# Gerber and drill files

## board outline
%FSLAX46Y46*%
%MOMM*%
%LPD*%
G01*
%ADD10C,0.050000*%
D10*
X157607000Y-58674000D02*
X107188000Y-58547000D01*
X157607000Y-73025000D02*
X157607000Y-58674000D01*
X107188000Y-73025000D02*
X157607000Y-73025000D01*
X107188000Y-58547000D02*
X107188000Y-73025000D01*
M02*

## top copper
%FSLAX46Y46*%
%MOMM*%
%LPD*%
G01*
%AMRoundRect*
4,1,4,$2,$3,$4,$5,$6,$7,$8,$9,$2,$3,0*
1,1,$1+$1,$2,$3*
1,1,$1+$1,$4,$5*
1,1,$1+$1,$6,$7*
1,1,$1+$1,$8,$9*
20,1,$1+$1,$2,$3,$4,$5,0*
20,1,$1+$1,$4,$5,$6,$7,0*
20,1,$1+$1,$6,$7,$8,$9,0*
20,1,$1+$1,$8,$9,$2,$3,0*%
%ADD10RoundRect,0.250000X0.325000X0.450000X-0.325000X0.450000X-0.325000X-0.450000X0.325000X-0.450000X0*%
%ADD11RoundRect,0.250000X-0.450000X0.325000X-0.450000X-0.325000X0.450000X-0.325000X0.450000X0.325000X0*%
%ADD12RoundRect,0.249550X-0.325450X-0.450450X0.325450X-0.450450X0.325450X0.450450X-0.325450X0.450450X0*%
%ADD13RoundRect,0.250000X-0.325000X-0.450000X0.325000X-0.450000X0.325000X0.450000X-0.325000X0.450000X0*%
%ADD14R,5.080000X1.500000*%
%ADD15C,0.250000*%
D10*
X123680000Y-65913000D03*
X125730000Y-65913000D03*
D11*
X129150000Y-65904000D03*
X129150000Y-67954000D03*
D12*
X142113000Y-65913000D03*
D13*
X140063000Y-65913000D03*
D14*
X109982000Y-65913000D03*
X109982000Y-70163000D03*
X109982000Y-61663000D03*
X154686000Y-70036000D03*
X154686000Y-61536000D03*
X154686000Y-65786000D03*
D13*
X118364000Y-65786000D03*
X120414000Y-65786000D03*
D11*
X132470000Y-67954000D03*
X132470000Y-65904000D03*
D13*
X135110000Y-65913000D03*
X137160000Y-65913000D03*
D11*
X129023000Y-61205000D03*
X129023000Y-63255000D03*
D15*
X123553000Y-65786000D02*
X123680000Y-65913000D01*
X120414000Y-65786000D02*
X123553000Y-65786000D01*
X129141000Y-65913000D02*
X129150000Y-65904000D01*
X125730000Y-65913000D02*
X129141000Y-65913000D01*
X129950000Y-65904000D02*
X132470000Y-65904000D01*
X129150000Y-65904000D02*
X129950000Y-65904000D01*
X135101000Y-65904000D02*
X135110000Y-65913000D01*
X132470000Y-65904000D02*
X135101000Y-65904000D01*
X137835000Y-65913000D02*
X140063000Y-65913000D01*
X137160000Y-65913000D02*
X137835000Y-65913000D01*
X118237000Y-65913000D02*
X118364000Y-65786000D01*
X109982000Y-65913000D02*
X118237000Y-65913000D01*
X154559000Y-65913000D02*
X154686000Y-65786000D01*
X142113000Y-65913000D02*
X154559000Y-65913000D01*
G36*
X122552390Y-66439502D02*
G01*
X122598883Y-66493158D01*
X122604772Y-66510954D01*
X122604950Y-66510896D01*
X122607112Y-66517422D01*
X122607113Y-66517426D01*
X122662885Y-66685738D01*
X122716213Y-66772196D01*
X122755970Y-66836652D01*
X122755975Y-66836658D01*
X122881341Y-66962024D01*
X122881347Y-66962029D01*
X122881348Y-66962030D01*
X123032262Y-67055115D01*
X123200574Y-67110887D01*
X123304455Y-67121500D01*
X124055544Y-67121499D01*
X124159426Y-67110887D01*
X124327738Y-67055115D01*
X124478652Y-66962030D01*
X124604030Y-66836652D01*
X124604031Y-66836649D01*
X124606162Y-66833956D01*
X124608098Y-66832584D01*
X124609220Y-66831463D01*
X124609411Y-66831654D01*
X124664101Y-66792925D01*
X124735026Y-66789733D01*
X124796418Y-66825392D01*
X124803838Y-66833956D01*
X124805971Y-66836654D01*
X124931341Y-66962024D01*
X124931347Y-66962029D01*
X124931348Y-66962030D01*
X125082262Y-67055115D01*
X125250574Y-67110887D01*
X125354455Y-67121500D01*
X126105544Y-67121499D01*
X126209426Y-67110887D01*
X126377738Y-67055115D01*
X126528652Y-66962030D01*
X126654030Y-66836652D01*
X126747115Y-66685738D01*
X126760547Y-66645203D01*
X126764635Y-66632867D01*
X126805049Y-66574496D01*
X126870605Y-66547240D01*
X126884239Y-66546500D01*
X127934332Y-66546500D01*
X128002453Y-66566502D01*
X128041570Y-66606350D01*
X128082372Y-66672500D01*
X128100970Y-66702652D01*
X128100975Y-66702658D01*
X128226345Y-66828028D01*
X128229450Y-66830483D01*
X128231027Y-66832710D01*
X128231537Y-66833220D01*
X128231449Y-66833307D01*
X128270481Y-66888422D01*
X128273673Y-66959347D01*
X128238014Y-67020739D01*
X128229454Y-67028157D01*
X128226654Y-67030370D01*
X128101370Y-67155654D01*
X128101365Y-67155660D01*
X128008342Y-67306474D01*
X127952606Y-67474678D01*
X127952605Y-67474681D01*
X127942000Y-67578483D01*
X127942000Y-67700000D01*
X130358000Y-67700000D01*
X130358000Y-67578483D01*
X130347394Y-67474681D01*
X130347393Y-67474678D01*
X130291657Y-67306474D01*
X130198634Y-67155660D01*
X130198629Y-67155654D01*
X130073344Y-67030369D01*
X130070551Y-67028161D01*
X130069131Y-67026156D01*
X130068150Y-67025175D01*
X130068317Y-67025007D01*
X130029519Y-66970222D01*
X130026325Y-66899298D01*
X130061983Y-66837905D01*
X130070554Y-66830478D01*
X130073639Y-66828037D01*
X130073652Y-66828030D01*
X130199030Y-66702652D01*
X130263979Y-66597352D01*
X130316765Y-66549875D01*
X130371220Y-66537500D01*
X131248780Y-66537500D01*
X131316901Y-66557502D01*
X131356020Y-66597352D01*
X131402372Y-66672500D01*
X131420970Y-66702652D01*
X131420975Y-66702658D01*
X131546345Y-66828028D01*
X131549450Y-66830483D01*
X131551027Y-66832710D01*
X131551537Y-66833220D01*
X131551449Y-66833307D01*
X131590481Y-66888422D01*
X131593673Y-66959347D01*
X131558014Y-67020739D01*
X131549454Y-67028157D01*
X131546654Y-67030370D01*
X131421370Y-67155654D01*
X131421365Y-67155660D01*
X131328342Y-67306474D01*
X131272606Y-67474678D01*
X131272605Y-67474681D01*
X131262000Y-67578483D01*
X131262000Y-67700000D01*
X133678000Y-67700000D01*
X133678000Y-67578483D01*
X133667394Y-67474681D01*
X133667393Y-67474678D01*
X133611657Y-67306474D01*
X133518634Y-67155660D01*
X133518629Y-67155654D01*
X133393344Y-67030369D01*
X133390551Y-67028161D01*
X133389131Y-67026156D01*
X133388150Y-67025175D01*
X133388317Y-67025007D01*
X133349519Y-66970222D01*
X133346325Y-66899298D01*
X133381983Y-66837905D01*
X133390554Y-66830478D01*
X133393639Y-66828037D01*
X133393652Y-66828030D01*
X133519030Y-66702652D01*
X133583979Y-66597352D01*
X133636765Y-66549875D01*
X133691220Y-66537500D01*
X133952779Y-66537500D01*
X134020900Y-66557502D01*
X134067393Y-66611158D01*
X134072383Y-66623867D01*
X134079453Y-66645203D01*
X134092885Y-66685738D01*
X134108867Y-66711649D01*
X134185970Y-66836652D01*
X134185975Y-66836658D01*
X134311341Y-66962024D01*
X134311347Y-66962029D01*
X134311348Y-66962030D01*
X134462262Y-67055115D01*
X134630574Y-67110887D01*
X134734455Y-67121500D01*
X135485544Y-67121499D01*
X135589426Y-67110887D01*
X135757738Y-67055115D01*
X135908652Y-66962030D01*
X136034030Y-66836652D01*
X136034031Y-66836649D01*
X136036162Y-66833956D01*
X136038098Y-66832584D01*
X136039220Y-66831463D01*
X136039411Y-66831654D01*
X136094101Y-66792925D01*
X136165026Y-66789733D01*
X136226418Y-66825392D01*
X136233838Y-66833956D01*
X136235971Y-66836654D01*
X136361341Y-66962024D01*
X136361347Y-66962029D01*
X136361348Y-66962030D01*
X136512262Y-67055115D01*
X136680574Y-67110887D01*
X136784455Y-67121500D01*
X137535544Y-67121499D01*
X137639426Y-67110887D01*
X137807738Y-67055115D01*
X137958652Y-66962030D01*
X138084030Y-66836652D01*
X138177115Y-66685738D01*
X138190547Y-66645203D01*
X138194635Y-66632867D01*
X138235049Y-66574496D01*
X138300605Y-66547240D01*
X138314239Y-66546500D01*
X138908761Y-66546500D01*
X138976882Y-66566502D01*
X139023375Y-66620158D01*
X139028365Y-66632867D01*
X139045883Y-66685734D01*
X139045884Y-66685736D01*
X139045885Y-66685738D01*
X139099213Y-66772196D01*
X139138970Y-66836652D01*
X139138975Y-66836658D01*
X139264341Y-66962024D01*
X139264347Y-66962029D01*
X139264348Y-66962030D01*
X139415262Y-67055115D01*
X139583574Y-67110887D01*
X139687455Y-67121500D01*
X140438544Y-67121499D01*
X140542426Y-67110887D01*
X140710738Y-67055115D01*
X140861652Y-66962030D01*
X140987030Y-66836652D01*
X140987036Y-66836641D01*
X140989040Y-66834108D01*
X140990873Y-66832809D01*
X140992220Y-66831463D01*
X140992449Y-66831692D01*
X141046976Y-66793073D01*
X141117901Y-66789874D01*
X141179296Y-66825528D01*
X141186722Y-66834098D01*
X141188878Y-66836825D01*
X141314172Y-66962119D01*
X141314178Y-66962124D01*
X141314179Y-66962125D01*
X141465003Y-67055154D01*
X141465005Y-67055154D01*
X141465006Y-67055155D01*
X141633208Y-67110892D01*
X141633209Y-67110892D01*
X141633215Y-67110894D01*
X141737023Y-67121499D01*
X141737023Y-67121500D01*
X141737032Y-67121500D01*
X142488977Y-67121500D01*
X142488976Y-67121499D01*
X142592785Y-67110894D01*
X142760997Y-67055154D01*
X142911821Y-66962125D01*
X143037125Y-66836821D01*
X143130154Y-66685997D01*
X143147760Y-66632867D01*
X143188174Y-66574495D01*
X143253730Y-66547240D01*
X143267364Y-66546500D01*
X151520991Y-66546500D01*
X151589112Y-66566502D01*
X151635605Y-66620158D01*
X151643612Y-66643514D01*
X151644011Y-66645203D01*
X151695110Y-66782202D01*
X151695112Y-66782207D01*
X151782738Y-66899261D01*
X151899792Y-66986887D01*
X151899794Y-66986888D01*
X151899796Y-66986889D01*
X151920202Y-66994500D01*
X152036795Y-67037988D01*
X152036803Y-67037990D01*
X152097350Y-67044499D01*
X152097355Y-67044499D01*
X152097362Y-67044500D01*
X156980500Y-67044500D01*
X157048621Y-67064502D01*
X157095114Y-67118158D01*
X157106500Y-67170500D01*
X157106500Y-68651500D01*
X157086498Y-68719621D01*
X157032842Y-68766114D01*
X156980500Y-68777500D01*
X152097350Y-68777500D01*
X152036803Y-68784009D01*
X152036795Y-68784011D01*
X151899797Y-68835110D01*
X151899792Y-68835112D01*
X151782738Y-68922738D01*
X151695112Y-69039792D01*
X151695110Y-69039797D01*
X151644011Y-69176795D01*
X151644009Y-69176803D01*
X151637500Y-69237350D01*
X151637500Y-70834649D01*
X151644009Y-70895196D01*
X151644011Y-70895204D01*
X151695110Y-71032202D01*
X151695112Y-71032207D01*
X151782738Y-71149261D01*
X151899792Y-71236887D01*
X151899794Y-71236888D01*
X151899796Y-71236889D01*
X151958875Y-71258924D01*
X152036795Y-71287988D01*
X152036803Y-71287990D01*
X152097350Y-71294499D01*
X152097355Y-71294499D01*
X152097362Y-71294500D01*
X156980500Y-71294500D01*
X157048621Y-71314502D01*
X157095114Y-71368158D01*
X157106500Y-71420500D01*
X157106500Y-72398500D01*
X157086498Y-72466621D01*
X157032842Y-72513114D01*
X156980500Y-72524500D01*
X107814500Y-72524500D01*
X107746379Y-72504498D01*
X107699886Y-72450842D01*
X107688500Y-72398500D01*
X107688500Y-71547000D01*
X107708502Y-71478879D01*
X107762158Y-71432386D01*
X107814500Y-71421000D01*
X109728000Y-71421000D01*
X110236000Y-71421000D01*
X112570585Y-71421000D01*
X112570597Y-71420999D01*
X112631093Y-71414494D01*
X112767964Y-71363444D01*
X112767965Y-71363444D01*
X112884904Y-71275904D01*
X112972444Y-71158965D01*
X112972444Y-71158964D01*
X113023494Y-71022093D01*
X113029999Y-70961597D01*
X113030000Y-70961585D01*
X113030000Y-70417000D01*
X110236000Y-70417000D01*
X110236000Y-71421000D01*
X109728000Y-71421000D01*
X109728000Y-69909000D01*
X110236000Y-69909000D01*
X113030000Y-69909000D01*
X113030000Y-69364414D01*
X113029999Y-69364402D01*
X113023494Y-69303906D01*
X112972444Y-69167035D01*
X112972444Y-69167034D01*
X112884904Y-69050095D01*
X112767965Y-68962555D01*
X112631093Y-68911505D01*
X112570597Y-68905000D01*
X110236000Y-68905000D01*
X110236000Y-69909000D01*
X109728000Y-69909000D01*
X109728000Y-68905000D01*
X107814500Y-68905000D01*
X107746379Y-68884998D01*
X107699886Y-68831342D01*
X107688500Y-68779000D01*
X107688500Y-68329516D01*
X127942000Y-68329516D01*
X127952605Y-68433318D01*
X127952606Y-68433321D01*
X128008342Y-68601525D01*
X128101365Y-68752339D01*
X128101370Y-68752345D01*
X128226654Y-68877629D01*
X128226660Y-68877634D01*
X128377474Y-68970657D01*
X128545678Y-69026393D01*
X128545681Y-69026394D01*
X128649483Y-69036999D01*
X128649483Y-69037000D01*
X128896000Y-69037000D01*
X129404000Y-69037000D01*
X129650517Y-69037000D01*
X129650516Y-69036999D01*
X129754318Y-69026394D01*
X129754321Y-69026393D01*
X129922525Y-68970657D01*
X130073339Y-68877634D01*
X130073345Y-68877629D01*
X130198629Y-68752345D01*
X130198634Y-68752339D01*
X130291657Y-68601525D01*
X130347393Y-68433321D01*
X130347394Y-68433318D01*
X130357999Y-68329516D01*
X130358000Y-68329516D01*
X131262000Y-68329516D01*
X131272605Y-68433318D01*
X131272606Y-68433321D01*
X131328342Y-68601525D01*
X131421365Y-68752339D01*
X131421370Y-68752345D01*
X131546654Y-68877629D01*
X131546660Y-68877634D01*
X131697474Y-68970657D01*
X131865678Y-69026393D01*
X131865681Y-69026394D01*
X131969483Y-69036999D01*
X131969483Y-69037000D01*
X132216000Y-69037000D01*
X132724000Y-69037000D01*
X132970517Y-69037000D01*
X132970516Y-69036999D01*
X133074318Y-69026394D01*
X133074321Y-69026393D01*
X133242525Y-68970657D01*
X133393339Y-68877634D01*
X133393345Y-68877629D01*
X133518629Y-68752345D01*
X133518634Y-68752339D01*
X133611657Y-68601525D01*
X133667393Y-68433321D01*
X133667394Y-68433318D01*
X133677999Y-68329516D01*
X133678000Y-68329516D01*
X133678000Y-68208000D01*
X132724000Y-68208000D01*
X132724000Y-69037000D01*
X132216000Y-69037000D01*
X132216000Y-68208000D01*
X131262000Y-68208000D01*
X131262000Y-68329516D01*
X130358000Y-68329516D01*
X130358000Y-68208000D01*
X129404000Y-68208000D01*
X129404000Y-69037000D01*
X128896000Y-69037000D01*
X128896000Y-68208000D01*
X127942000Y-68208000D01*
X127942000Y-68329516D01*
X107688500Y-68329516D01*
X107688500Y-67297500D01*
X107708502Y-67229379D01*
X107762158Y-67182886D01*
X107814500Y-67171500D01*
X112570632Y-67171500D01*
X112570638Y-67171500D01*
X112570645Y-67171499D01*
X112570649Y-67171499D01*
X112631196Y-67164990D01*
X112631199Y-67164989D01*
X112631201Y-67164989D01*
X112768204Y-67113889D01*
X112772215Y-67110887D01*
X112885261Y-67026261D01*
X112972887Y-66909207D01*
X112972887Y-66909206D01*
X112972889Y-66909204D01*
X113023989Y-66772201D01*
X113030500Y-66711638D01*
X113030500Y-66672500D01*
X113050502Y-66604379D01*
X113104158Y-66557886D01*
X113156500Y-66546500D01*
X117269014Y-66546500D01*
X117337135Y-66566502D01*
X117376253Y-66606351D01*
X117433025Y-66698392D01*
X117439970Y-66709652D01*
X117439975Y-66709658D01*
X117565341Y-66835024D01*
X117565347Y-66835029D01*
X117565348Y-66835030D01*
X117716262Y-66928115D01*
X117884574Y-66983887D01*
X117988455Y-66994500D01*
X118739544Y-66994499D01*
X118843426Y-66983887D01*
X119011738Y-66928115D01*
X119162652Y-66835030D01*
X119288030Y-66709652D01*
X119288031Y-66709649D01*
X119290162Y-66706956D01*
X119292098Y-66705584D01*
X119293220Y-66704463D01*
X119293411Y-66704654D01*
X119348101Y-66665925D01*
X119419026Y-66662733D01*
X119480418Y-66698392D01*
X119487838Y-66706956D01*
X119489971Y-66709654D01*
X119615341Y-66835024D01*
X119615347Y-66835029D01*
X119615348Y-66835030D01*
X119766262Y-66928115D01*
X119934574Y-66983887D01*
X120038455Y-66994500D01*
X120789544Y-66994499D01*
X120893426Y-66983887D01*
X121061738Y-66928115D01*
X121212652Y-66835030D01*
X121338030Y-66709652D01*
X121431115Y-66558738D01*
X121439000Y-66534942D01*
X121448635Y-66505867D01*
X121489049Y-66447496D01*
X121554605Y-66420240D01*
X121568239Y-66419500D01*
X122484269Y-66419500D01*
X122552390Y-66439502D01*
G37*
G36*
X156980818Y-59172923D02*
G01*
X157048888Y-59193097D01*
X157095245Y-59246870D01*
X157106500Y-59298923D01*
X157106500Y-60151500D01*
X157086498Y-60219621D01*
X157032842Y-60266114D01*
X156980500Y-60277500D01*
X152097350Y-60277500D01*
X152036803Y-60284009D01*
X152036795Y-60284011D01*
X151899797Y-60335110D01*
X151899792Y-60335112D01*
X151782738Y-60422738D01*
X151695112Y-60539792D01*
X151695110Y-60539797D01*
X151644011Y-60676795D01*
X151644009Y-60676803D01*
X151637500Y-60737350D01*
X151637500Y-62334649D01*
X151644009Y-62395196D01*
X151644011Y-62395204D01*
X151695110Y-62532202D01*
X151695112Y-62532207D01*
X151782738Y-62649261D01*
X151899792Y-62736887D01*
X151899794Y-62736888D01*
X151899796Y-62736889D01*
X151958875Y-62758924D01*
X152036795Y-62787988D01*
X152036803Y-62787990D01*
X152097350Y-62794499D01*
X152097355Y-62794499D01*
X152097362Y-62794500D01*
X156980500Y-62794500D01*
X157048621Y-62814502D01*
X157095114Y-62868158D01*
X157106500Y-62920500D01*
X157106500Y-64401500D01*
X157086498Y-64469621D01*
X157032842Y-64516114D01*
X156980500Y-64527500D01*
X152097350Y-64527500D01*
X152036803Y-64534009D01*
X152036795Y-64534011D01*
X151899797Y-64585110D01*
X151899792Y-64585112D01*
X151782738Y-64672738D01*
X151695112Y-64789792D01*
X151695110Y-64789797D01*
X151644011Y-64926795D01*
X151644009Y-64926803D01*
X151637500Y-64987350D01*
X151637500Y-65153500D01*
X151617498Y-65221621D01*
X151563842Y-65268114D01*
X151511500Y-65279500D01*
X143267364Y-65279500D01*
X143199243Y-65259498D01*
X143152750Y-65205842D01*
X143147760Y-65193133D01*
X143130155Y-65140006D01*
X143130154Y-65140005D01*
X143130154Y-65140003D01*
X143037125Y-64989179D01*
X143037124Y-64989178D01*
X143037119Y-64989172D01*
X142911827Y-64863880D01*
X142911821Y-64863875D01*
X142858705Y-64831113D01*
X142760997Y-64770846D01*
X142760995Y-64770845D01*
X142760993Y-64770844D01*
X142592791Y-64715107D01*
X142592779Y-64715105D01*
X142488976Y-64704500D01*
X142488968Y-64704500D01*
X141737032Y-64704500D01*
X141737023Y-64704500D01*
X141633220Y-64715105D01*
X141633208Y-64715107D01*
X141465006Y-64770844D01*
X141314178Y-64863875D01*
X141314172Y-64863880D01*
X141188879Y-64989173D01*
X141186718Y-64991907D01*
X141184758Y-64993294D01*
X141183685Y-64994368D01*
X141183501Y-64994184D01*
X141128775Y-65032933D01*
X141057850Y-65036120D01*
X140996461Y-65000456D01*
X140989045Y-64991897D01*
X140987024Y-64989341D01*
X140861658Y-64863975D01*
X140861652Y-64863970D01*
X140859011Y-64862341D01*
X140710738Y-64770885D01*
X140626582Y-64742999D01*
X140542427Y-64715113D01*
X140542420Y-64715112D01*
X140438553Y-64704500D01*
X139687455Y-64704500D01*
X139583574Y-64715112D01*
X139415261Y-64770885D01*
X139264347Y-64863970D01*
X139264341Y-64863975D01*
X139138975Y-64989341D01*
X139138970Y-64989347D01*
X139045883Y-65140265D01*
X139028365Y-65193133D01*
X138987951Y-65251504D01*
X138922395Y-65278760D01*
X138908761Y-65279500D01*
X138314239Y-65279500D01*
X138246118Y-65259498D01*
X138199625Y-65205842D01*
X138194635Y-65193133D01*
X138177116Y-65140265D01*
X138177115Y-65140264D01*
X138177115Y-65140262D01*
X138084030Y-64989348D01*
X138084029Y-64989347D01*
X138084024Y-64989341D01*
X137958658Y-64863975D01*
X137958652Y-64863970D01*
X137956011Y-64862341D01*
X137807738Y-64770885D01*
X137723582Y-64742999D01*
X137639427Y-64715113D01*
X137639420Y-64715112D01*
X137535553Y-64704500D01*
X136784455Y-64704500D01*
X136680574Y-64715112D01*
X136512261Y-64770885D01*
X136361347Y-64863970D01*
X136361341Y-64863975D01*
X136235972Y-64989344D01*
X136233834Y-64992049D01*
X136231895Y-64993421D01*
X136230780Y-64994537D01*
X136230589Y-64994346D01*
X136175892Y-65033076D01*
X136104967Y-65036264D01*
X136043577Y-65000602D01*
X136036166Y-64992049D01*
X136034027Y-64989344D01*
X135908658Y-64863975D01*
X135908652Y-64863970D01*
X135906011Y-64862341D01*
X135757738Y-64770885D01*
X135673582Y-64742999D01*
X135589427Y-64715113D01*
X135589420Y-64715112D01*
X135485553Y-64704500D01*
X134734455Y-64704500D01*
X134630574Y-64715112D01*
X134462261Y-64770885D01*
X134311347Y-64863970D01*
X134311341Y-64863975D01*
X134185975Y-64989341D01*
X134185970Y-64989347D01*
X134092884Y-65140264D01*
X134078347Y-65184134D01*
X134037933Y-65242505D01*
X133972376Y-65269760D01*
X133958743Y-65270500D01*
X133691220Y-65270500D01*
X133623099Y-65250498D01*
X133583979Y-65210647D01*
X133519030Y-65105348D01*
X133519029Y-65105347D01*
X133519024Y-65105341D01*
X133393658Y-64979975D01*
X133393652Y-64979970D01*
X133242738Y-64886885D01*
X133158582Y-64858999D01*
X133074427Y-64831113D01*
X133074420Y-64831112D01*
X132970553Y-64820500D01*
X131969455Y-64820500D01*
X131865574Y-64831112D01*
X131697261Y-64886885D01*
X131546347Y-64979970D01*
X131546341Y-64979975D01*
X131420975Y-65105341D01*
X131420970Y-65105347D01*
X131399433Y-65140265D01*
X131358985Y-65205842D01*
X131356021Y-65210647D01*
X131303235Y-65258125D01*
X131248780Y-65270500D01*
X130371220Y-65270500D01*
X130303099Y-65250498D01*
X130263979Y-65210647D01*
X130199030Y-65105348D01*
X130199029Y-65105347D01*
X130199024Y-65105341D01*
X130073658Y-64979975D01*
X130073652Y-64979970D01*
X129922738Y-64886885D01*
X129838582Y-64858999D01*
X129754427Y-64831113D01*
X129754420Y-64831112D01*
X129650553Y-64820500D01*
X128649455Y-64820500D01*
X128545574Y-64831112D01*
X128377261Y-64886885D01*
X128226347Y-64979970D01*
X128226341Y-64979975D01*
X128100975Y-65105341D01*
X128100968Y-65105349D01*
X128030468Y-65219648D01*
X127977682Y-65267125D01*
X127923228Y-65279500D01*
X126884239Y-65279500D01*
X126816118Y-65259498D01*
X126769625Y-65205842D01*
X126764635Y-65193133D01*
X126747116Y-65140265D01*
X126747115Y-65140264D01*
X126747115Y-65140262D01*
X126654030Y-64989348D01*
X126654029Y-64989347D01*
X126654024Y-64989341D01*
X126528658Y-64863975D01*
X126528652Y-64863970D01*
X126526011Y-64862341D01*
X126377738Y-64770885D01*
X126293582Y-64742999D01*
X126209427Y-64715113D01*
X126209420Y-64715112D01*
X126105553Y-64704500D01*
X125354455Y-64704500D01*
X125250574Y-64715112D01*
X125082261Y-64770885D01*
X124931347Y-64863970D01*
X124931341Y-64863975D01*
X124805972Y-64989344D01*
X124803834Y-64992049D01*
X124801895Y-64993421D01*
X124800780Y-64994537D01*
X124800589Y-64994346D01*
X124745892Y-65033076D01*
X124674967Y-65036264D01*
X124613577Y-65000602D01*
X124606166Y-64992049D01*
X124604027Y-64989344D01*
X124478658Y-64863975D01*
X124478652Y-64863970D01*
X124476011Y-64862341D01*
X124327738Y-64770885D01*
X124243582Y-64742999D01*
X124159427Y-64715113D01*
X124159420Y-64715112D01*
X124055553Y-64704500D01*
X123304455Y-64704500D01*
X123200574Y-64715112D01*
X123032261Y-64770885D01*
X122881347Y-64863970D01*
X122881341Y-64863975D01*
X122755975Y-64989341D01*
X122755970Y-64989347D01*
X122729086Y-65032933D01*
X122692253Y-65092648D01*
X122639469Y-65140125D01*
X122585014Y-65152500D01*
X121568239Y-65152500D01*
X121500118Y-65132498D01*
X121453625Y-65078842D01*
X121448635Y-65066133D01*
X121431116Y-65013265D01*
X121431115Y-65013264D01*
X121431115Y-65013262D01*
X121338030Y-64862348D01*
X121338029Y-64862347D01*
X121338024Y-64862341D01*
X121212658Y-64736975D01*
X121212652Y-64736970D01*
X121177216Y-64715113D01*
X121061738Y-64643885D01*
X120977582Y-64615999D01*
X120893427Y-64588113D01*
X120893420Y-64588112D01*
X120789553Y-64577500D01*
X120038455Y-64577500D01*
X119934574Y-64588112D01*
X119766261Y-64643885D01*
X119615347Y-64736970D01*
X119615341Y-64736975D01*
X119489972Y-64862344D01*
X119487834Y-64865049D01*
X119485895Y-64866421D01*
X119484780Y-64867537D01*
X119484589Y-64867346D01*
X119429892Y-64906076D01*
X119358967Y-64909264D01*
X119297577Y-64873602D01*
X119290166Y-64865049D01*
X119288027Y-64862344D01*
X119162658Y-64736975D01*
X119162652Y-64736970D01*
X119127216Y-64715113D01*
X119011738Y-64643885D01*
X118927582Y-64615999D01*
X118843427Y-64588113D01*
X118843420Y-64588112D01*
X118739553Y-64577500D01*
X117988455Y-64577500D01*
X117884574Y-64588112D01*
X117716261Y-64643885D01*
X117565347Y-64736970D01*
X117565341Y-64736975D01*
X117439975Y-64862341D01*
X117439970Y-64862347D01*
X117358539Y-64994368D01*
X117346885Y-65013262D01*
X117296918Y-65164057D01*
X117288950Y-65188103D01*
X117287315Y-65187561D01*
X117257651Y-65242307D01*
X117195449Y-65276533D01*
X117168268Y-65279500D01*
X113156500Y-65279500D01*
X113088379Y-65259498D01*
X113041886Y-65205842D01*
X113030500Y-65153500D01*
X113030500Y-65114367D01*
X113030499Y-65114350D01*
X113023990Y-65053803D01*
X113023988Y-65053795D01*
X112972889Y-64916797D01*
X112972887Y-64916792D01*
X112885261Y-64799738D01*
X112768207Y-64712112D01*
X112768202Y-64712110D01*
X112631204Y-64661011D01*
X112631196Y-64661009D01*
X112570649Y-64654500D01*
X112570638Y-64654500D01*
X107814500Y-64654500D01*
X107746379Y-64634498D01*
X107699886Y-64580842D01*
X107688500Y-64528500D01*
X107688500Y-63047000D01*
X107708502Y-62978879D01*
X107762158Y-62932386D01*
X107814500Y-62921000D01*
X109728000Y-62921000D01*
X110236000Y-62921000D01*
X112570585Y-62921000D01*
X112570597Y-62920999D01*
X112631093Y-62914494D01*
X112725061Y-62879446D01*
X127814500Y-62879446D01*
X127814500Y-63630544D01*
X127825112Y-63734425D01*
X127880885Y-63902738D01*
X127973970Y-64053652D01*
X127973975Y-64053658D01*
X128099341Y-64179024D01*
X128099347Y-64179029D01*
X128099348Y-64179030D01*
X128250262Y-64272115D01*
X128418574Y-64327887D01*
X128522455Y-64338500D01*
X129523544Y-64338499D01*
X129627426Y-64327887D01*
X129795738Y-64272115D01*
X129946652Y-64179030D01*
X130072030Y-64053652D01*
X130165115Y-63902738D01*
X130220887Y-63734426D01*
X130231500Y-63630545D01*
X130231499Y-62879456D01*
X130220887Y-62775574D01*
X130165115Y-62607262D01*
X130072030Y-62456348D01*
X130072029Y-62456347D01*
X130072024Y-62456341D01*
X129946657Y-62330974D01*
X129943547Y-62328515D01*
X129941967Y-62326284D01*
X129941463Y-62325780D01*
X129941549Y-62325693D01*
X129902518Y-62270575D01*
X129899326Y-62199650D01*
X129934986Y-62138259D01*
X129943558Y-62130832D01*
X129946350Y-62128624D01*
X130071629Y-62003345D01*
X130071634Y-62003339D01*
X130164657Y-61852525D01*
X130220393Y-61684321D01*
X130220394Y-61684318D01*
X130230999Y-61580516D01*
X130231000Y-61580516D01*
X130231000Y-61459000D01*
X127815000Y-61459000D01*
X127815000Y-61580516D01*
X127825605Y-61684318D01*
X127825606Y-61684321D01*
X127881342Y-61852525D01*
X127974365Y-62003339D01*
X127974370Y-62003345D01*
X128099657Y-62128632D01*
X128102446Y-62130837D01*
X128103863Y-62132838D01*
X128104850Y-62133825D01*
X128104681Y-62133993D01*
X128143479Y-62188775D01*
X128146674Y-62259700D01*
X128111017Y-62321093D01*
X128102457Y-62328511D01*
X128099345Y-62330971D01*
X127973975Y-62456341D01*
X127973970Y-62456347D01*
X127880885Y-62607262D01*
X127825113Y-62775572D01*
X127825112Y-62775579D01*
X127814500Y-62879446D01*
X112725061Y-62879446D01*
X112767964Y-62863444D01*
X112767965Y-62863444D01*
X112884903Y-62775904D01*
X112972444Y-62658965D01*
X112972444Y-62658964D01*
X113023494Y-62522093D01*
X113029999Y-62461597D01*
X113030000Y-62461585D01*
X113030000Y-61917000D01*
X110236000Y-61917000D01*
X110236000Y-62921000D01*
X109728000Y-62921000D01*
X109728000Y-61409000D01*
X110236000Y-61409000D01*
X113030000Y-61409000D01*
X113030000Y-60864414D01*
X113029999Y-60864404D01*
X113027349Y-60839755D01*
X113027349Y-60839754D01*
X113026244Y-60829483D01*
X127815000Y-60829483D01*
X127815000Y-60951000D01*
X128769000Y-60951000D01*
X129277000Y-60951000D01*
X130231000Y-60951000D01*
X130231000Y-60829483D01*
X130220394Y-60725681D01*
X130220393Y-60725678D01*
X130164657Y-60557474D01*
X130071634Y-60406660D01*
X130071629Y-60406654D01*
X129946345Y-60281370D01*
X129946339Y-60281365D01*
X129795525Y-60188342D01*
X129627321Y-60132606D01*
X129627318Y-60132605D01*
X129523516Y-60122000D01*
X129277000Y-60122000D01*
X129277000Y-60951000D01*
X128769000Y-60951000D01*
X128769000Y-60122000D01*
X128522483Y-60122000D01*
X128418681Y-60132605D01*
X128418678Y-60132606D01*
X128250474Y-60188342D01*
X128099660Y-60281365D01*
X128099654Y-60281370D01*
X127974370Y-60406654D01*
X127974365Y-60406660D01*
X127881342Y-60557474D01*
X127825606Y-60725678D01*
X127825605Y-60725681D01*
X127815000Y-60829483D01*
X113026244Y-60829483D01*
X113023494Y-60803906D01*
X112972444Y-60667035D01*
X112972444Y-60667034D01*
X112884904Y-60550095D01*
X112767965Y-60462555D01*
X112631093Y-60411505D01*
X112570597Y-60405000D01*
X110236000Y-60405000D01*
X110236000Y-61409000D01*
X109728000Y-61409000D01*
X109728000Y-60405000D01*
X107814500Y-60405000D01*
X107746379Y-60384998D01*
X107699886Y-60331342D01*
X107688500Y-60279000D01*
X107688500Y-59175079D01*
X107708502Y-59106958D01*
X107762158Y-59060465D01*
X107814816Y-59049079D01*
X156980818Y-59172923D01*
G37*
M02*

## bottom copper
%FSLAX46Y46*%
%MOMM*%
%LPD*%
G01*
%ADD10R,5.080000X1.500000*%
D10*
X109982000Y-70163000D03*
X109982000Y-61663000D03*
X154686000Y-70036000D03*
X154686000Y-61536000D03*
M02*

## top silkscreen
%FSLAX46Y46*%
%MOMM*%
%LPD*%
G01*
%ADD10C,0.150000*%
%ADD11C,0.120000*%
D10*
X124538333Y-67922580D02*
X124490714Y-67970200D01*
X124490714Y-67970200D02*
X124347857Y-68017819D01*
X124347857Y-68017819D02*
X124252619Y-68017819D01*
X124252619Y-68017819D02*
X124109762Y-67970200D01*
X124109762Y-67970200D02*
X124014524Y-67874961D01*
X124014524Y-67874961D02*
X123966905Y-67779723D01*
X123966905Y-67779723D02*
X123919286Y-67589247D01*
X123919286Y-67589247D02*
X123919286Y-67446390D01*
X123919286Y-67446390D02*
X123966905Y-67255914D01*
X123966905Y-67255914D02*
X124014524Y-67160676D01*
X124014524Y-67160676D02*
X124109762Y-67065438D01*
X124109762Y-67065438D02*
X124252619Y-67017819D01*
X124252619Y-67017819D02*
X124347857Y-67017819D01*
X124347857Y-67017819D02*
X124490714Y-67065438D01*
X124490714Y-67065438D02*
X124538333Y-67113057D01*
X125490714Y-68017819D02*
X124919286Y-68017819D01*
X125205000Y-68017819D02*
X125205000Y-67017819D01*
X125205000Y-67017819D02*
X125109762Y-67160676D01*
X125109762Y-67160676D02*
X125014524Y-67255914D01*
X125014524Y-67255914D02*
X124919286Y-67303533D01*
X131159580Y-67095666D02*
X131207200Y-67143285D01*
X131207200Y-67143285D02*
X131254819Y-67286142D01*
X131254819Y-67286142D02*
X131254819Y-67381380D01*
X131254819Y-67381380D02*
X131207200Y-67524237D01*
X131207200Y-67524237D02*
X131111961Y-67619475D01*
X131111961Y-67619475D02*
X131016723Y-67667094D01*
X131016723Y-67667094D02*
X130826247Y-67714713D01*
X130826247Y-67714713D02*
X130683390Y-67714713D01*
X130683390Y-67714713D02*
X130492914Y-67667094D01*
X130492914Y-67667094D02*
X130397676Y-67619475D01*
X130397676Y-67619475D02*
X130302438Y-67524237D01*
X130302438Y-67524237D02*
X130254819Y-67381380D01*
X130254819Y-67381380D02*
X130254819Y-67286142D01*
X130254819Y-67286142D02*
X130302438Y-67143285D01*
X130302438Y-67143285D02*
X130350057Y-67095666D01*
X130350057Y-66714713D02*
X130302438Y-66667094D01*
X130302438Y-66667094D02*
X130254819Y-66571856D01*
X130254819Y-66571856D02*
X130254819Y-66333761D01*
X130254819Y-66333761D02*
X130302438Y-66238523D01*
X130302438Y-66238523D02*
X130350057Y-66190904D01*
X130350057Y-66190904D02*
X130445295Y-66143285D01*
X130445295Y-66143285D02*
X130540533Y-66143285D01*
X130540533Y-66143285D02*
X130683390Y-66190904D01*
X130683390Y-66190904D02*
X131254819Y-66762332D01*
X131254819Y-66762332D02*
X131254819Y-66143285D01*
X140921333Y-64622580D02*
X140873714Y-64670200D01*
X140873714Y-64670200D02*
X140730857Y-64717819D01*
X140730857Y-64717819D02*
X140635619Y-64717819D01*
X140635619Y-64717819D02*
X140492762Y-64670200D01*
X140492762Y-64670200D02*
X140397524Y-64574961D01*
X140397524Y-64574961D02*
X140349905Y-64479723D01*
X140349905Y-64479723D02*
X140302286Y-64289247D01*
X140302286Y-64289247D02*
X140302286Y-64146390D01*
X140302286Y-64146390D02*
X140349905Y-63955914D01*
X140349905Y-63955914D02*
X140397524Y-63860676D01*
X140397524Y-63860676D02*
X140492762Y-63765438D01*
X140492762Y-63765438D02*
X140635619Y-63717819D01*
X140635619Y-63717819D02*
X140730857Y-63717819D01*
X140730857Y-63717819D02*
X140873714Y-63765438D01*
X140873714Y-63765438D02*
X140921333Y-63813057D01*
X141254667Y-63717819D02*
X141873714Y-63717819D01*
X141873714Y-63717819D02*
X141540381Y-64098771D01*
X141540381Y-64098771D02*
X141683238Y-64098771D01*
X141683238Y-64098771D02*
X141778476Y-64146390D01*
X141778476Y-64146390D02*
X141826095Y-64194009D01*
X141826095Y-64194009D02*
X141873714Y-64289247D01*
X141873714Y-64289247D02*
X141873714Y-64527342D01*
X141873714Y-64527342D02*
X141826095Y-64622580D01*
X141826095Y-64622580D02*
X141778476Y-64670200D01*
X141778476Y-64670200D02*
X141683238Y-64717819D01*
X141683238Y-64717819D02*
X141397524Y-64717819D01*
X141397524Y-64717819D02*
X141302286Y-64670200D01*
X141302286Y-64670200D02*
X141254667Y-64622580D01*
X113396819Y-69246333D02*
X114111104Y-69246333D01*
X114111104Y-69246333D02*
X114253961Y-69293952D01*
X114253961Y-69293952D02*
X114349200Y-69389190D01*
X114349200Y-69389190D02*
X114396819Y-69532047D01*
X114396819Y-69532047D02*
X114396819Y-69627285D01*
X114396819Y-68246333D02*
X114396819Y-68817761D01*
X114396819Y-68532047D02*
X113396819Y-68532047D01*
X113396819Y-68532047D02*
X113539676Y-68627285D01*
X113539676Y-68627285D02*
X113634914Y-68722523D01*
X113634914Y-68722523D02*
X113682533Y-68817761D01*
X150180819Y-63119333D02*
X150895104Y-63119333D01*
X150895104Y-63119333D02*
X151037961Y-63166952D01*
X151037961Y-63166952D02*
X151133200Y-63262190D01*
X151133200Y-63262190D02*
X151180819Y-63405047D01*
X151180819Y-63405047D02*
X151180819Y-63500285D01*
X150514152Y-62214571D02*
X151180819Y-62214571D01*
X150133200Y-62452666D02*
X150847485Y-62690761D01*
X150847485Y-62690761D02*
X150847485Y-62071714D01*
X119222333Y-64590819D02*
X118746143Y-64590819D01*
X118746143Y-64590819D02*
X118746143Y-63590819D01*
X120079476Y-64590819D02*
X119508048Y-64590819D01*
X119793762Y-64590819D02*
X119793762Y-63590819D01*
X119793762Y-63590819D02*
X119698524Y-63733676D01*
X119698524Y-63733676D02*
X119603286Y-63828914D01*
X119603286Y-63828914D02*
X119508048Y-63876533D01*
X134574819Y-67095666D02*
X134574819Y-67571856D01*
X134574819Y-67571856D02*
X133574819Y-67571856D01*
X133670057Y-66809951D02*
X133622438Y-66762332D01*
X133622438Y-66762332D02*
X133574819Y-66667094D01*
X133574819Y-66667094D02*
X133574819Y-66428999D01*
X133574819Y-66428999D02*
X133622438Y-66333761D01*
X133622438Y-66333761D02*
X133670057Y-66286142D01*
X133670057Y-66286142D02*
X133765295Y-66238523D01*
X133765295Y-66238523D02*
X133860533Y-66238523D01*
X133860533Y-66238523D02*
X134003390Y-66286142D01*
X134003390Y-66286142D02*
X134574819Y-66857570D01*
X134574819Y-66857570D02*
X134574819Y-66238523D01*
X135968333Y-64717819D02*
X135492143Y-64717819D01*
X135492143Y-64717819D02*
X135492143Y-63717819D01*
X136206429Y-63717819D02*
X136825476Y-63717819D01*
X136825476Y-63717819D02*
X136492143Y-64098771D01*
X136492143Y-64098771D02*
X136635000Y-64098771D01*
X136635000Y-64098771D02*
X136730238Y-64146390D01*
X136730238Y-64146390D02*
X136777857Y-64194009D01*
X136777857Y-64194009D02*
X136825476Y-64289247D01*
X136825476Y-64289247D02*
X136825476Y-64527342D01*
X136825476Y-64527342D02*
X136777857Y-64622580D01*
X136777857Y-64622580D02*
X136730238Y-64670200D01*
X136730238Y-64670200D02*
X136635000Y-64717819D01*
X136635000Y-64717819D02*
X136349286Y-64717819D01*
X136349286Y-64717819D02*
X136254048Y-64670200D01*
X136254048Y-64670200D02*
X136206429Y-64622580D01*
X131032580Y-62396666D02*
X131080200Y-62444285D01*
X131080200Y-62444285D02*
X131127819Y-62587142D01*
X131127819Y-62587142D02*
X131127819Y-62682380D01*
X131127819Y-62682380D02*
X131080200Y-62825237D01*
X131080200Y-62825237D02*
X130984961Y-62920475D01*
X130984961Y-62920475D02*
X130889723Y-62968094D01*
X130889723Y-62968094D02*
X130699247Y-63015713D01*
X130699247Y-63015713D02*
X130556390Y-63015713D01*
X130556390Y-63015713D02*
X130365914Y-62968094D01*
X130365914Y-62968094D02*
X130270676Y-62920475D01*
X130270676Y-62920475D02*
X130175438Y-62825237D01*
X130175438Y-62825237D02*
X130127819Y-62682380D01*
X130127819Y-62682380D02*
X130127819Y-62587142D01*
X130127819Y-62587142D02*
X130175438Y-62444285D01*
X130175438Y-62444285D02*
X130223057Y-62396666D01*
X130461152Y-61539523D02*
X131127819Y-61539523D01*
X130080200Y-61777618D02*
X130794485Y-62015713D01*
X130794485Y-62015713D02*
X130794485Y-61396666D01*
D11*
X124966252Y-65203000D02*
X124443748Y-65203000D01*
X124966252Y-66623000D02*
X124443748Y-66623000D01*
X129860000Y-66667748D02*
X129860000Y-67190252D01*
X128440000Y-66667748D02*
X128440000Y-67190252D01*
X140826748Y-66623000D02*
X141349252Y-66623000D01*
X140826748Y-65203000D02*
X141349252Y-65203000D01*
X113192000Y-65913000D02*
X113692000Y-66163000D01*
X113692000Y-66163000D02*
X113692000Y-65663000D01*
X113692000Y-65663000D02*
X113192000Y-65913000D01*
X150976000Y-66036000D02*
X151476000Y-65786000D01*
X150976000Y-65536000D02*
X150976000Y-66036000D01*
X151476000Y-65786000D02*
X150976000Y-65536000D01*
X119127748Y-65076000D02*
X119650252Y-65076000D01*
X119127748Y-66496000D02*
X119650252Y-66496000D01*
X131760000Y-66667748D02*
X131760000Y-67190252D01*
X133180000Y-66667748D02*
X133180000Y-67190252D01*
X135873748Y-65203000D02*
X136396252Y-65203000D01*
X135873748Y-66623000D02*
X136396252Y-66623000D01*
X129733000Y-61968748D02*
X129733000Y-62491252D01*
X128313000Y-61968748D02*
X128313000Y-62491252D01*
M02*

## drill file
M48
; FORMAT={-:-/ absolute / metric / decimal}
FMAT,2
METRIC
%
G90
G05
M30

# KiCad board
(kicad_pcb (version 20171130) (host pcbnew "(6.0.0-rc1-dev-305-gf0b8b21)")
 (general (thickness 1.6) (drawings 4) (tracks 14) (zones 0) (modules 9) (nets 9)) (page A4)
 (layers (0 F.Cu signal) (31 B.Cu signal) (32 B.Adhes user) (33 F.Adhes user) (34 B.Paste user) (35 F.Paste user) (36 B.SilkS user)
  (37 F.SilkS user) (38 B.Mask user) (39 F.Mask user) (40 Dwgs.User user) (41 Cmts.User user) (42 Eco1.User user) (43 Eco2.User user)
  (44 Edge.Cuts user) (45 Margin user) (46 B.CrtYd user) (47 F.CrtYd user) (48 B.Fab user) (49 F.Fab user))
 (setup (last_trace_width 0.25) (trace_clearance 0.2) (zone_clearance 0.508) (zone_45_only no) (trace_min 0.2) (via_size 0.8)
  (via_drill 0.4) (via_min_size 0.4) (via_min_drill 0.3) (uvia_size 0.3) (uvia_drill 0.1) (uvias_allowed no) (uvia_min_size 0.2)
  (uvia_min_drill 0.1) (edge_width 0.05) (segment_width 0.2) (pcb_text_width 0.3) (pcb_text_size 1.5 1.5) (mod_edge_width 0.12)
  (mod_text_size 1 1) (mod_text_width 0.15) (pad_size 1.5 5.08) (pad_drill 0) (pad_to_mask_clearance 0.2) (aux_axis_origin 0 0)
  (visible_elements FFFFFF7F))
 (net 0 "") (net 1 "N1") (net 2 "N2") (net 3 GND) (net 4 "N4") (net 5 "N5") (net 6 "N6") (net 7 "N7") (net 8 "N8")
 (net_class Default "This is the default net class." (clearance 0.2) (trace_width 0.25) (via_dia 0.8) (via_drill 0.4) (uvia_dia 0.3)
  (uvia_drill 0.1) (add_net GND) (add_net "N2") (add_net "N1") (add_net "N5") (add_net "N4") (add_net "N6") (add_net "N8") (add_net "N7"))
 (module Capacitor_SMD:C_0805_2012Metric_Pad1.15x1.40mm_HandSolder (layer F.Cu) (at 124.705 65.913 180)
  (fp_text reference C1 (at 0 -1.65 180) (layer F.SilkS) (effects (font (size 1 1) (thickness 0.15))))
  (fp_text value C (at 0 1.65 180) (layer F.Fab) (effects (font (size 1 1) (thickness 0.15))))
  (fp_line (start -0.261252 0.71) (end 0.261252 0.71) (layer F.SilkS) (width 0.12))
  (fp_line (start -0.261252 -0.71) (end 0.261252 -0.71) (layer F.SilkS) (width 0.12))
  (pad 2 smd roundrect (at 1.025 0 180) (size 1.15 1.4) (layers F.Cu F.Paste F.Mask) (roundrect_rratio 0.217391) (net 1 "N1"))
  (pad 1 smd roundrect (at -1.025 0 180) (size 1.15 1.4) (layers F.Cu F.Paste F.Mask) (roundrect_rratio 0.217391) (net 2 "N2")))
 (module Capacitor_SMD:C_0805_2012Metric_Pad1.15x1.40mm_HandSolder (layer F.Cu) (at 129.15 66.929 270)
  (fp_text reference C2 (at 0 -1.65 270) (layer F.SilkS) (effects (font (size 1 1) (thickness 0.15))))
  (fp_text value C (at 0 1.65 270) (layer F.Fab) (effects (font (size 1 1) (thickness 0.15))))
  (fp_line (start -0.261252 -0.71) (end 0.261252 -0.71) (layer F.SilkS) (width 0.12))
  (fp_line (start -0.261252 0.71) (end 0.261252 0.71) (layer F.SilkS) (width 0.12))
  (pad 1 smd roundrect (at -1.025 0 270) (size 1.15 1.4) (layers F.Cu F.Paste F.Mask) (roundrect_rratio 0.217391) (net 2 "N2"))
  (pad 2 smd roundrect (at 1.025 0 270) (size 1.15 1.4) (layers F.Cu F.Paste F.Mask) (roundrect_rratio 0.217391) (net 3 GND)))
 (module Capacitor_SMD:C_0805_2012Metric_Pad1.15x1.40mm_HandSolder (layer F.Cu) (at 141.088 65.913)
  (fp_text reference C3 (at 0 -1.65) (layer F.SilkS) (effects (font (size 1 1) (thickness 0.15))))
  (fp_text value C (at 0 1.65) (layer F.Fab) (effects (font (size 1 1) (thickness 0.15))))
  (fp_line (start -0.261252 0.71) (end 0.261252 0.71) (layer F.SilkS) (width 0.12))
  (fp_line (start -0.261252 -0.71) (end 0.261252 -0.71) (layer F.SilkS) (width 0.12))
  (pad 2 smd roundrect (at 1.025 0) (size 1.15 1.4) (layers F.Cu F.Paste F.Mask) (roundrect_rratio 0.217) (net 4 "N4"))
  (pad 1 smd roundrect (at -1.025 0) (size 1.15 1.4) (layers F.Cu F.Paste F.Mask) (roundrect_rratio 0.217391) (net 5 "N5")))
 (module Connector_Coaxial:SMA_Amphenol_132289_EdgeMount (layer F.Cu) (at 109.982 65.913 180)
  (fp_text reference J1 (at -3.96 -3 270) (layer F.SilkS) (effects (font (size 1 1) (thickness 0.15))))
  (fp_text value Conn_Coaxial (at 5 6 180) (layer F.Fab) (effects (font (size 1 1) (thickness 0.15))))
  (fp_line (start -3.21 0) (end -3.71 -0.25) (layer F.SilkS) (width 0.12))
  (fp_line (start -3.71 -0.25) (end -3.71 0.25) (layer F.SilkS) (width 0.12))
  (fp_line (start -3.71 0.25) (end -3.21 0) (layer F.SilkS) (width 0.12))
  (pad 1 smd rect (at 0 0 270) (size 1.5 5.08) (layers F.Cu F.Paste F.Mask) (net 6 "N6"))
  (pad 2 smd rect (at 0 -4.25 270) (size 1.5 5.08) (layers F.Cu F.Paste F.Mask) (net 3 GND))
  (pad 2 smd rect (at 0 4.25 270) (size 1.5 5.08) (layers F.Cu F.Paste F.Mask) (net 3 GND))
  (pad 2 smd rect (at 0 -4.25 270) (size 1.5 5.08) (layers B.Cu B.Paste B.Mask) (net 3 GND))
  (pad 2 smd rect (at 0 4.25 270) (size 1.5 5.08) (layers B.Cu B.Paste B.Mask) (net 3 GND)))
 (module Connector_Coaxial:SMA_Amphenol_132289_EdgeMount (layer F.Cu) (at 154.686 65.786)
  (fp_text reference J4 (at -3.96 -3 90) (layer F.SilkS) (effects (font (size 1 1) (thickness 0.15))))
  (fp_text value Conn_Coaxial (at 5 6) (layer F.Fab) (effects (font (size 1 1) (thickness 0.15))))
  (fp_line (start -3.71 0.25) (end -3.21 0) (layer F.SilkS) (width 0.12))
  (fp_line (start -3.71 -0.25) (end -3.71 0.25) (layer F.SilkS) (width 0.12))
  (fp_line (start -3.21 0) (end -3.71 -0.25) (layer F.SilkS) (width 0.12))
  (pad 2 smd rect (at 0 4.25 90) (size 1.5 5.08) (layers B.Cu B.Paste B.Mask) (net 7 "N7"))
  (pad 2 smd rect (at 0 -4.25 90) (size 1.5 5.08) (layers B.Cu B.Paste B.Mask) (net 7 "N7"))
  (pad 2 smd rect (at 0 4.25 90) (size 1.5 5.08) (layers F.Cu F.Paste F.Mask) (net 7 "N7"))
  (pad 2 smd rect (at 0 -4.25 90) (size 1.5 5.08) (layers F.Cu F.Paste F.Mask) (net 7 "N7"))
  (pad 1 smd rect (at 0 0 90) (size 1.5 5.08) (layers F.Cu F.Paste F.Mask) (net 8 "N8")))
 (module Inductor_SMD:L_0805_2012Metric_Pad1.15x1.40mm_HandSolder (layer F.Cu) (at 119.389 65.786)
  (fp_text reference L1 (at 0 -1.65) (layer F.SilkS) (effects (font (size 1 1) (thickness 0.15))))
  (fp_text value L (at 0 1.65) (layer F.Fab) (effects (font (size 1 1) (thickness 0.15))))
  (fp_line (start -0.261252 -0.71) (end 0.261252 -0.71) (layer F.SilkS) (width 0.12))
  (fp_line (start -0.261252 0.71) (end 0.261252 0.71) (layer F.SilkS) (width 0.12))
  (pad 1 smd roundrect (at -1.025 0) (size 1.15 1.4) (layers F.Cu F.Paste F.Mask) (roundrect_rratio 0.217391) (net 6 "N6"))
  (pad 2 smd roundrect (at 1.025 0) (size 1.15 1.4) (layers F.Cu F.Paste F.Mask) (roundrect_rratio 0.217391) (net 1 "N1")))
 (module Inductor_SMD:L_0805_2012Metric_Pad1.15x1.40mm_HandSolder (layer F.Cu) (at 132.47 66.929 270)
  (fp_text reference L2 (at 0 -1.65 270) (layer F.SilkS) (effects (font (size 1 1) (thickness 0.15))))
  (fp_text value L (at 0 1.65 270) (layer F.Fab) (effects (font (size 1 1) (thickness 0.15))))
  (fp_line (start -0.261252 0.71) (end 0.261252 0.71) (layer F.SilkS) (width 0.12))
  (fp_line (start -0.261252 -0.71) (end 0.261252 -0.71) (layer F.SilkS) (width 0.12))
  (pad 2 smd roundrect (at 1.025 0 270) (size 1.15 1.4) (layers F.Cu F.Paste F.Mask) (roundrect_rratio 0.217391) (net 3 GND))
  (pad 1 smd roundrect (at -1.025 0 270) (size 1.15 1.4) (layers F.Cu F.Paste F.Mask) (roundrect_rratio 0.217391) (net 2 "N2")))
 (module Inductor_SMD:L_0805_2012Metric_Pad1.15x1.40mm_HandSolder (layer F.Cu) (at 136.135 65.913)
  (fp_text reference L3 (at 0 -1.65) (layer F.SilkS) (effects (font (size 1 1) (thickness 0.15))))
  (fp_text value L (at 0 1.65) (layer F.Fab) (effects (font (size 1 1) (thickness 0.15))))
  (fp_line (start -0.261252 -0.71) (end 0.261252 -0.71) (layer F.SilkS) (width 0.12))
  (fp_line (start -0.261252 0.71) (end 0.261252 0.71) (layer F.SilkS) (width 0.12))
  (pad 1 smd roundrect (at -1.025 0) (size 1.15 1.4) (layers F.Cu F.Paste F.Mask) (roundrect_rratio 0.217391) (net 2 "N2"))
  (pad 2 smd roundrect (at 1.025 0) (size 1.15 1.4) (layers F.Cu F.Paste F.Mask) (roundrect_rratio 0.217391) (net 5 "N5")))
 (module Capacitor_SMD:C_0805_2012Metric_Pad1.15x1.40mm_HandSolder (layer F.Cu) (at 129.023 62.23 270)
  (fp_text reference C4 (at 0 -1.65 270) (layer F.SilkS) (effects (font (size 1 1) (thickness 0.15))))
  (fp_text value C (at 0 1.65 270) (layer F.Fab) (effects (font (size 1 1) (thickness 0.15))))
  (fp_line (start -0.261252 -0.71) (end 0.261252 -0.71) (layer F.SilkS) (width 0.12))
  (fp_line (start -0.261252 0.71) (end 0.261252 0.71) (layer F.SilkS) (width 0.12))
  (pad 1 smd roundrect (at -1.025 0 270) (size 1.15 1.4) (layers F.Cu F.Paste F.Mask) (roundrect_rratio 0.217391) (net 3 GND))
  (pad 2 smd roundrect (at 1.025 0 270) (size 1.15 1.4) (layers F.Cu F.Paste F.Mask) (roundrect_rratio 0.217391) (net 2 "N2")))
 (gr_line (start 157.607 58.674) (end 107.188 58.547) (layer Edge.Cuts) (width 0.05))
 (gr_line (start 157.607 73.025) (end 157.607 58.674) (layer Edge.Cuts) (width 0.05))
 (gr_line (start 107.188 73.025) (end 157.607 73.025) (layer Edge.Cuts) (width 0.05))
 (gr_line (start 107.188 58.547) (end 107.188 73.025) (layer Edge.Cuts) (width 0.05))
 (segment (start 123.553 65.786) (end 123.68 65.913) (width 0.25) (layer F.Cu) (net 1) (status 30))
 (segment (start 120.414 65.786) (end 123.553 65.786) (width 0.25) (layer F.Cu) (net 1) (status 30))
 (segment (start 129.141 65.913) (end 129.15 65.904) (width 0.25) (layer F.Cu) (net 2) (status 30))
 (segment (start 125.73 65.913) (end 129.141 65.913) (width 0.25) (layer F.Cu) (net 2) (status 30))
 (segment (start 129.95 65.904) (end 132.47 65.904) (width 0.25) (layer F.Cu) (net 2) (status 20))
 (segment (start 129.15 65.904) (end 129.95 65.904) (width 0.25) (layer F.Cu) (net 2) (status 10))
 (segment (start 135.101 65.904) (end 135.11 65.913) (width 0.25) (layer F.Cu) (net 2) (status 30))
 (segment (start 132.47 65.904) (end 135.101 65.904) (width 0.25) (layer F.Cu) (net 2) (status 30))
 (segment (start 137.835 65.913) (end 140.063 65.913) (width 0.25) (layer F.Cu) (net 5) (status 20))
 (segment (start 137.16 65.913) (end 137.835 65.913) (width 0.25) (layer F.Cu) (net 5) (status 10))
 (segment (start 118.237 65.913) (end 118.364 65.786) (width 0.25) (layer F.Cu) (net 6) (status 30))
 (segment (start 109.982 65.913) (end 118.237 65.913) (width 0.25) (layer F.Cu) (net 6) (status 30))
 (segment (start 154.559 65.913) (end 154.686 65.786) (width 0.25) (layer F.Cu) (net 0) (status 30))
 (segment (start 142.113 65.913) (end 154.559 65.913) (width 0.25) (layer F.Cu) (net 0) (status 30))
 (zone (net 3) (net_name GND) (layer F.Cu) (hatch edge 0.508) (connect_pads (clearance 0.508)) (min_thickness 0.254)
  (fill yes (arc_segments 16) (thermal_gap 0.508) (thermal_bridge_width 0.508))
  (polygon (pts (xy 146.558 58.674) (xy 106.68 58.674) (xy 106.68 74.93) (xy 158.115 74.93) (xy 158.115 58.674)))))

